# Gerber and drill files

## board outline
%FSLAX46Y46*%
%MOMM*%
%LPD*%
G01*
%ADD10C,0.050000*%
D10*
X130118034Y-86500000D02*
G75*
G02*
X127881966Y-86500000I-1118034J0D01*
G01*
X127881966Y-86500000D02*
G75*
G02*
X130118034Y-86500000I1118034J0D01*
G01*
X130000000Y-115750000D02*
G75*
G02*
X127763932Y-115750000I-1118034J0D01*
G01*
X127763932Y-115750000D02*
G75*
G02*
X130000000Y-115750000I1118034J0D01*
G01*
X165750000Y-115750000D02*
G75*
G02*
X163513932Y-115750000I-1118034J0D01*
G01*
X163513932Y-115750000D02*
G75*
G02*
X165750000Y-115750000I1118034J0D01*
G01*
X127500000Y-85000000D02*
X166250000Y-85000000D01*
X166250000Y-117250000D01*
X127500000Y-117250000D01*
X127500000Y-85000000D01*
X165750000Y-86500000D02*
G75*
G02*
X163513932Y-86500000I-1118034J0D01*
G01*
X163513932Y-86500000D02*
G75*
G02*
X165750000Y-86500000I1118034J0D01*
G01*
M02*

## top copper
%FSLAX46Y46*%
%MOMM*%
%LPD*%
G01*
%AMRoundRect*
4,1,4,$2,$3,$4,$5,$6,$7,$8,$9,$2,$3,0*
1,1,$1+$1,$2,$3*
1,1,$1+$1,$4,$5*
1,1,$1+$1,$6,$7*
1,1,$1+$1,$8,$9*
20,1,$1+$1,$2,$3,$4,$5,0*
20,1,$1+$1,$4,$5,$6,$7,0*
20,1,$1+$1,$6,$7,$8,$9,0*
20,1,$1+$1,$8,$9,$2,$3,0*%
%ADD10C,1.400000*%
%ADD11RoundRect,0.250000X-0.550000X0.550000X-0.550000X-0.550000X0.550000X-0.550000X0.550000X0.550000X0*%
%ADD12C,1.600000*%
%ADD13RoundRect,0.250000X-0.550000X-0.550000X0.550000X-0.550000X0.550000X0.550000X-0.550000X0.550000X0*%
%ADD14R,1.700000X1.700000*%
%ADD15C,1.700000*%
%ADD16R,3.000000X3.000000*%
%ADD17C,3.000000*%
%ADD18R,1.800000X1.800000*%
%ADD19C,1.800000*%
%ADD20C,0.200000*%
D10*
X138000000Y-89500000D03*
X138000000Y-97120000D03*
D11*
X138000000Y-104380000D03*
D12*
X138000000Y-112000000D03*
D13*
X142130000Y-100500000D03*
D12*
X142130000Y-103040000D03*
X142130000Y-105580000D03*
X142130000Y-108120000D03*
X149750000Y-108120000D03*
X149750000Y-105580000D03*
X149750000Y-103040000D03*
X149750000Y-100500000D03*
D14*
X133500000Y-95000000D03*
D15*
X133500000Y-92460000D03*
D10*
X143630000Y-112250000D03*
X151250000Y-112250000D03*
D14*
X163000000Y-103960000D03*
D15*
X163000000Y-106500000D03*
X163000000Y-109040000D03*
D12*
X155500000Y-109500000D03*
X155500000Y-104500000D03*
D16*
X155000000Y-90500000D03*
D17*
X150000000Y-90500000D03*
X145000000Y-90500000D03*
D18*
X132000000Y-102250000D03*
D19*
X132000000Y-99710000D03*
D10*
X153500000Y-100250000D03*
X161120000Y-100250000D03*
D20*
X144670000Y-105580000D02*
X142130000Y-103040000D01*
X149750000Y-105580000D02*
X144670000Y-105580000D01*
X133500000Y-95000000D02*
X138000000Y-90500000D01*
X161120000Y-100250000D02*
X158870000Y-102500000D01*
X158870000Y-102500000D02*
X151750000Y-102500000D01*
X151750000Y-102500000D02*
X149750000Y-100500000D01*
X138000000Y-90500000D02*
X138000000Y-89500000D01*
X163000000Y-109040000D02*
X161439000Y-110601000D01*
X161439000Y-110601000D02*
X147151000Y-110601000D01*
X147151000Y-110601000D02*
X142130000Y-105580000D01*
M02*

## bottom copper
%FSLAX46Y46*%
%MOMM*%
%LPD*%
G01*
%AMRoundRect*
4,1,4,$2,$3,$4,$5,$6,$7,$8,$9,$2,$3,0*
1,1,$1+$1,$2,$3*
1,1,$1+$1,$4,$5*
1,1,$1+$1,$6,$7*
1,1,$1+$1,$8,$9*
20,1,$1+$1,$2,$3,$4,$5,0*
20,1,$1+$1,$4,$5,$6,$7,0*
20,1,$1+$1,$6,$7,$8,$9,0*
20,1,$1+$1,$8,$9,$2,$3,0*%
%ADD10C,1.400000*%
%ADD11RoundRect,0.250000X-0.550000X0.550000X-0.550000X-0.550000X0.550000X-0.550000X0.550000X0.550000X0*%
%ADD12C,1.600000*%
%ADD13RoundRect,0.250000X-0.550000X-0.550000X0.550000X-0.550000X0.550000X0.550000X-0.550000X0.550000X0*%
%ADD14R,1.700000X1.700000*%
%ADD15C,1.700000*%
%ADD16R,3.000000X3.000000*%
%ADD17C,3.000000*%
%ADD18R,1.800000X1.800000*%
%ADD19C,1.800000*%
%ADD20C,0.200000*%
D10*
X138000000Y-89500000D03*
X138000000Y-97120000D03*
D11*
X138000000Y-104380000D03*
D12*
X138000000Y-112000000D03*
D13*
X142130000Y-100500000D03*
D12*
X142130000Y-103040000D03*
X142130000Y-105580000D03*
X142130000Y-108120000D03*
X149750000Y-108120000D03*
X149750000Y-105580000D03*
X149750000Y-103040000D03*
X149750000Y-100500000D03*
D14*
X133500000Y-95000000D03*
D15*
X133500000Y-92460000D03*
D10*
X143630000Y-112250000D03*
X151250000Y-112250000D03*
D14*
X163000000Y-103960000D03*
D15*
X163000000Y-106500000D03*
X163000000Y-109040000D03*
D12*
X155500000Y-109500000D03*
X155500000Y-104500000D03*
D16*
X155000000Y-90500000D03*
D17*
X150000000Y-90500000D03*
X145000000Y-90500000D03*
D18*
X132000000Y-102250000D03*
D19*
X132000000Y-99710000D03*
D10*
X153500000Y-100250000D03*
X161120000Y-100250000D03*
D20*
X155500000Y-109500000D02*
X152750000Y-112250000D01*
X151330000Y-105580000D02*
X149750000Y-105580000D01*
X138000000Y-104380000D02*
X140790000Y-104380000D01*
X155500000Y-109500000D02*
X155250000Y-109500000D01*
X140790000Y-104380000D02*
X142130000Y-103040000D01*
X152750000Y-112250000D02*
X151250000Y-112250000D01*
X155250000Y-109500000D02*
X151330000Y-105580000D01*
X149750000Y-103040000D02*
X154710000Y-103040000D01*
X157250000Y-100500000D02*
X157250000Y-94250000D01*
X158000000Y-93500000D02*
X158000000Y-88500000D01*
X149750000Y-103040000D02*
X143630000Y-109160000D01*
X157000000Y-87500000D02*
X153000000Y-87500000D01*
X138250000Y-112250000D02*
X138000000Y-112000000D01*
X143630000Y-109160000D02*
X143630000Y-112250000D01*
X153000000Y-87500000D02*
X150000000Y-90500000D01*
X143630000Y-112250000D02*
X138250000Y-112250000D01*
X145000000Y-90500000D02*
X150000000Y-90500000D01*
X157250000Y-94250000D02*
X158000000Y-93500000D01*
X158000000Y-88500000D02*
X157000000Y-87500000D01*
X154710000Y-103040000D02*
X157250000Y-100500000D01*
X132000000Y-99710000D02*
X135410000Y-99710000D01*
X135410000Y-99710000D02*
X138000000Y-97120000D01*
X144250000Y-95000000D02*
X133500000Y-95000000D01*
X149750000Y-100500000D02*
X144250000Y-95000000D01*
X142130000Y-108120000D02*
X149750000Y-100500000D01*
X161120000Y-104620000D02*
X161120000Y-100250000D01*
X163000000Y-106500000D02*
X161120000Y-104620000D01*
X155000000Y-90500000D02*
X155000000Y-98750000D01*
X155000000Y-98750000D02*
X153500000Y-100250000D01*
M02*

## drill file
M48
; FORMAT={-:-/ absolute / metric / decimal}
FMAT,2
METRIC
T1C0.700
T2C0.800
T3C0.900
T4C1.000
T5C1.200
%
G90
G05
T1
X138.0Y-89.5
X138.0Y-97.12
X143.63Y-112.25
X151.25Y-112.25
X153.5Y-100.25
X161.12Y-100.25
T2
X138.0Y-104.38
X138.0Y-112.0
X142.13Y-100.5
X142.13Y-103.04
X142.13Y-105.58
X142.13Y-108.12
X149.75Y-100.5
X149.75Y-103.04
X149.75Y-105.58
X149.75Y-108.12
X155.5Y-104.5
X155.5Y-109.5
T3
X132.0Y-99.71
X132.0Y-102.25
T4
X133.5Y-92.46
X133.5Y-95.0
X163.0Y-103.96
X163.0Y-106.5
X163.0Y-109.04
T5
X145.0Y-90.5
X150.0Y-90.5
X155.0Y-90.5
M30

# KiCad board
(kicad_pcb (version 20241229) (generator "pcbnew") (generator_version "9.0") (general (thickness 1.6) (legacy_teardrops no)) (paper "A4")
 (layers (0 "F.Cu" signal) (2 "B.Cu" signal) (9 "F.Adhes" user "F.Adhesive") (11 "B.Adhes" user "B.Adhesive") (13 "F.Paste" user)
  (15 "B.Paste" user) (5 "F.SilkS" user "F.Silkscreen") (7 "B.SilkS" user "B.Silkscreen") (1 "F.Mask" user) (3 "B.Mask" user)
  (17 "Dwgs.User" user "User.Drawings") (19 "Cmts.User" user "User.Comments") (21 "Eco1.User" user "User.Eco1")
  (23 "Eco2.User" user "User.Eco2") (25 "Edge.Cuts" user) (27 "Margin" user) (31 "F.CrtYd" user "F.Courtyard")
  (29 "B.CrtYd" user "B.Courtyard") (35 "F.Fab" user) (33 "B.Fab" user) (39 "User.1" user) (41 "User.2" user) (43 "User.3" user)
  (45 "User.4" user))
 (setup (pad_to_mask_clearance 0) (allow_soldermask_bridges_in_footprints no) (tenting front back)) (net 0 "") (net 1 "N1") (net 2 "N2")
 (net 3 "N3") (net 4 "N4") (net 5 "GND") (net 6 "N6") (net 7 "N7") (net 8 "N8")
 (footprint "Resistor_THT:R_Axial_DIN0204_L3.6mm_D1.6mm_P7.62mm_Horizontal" (layer "F.Cu") (at 138 89.5 -90)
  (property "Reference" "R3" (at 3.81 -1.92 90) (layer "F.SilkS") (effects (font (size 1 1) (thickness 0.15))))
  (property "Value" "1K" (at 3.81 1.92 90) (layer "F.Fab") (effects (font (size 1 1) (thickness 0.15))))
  (pad "1" thru_hole circle (at 0 0 270) (size 1.4 1.4) (drill 0.7) (layers "*.Cu" "*.Mask") (remove_unused_layers no) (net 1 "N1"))
  (pad "2" thru_hole circle (at 7.62 0 270) (size 1.4 1.4) (drill 0.7) (layers "*.Cu" "*.Mask") (remove_unused_layers no) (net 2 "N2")))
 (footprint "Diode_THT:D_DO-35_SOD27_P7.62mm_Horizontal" (layer "F.Cu") (at 138 104.38 -90)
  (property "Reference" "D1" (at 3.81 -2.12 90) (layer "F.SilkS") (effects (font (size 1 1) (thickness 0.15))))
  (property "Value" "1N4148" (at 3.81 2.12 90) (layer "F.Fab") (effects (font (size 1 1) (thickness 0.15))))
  (pad "1" thru_hole roundrect (at 0 0 270) (size 1.6 1.6) (drill 0.8) (layers "*.Cu" "*.Mask") (remove_unused_layers no)
   (roundrect_rratio 0.15625) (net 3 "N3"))
  (pad "2" thru_hole circle (at 7.62 0 270) (size 1.6 1.6) (drill 0.8) (layers "*.Cu" "*.Mask") (remove_unused_layers no) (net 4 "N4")))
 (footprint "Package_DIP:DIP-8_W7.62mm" (layer "F.Cu") (at 142.13 100.5)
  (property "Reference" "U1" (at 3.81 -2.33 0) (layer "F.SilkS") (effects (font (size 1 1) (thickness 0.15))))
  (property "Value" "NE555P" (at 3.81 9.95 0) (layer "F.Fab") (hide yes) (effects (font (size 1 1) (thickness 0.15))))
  (pad "1" thru_hole roundrect (at 0 0) (size 1.6 1.6) (drill 0.8) (layers "*.Cu" "*.Mask") (remove_unused_layers no)
   (roundrect_rratio 0.15625) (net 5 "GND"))
  (pad "2" thru_hole circle (at 0 2.54) (size 1.6 1.6) (drill 0.8) (layers "*.Cu" "*.Mask") (remove_unused_layers no) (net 3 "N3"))
  (pad "3" thru_hole circle (at 0 5.08) (size 1.6 1.6) (drill 0.8) (layers "*.Cu" "*.Mask") (remove_unused_layers no) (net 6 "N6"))
  (pad "4" thru_hole circle (at 0 7.62) (size 1.6 1.6) (drill 0.8) (layers "*.Cu" "*.Mask") (remove_unused_layers no) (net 1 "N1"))
  (pad "5" thru_hole circle (at 7.62 7.62) (size 1.6 1.6) (drill 0.8) (layers "*.Cu" "*.Mask") (remove_unused_layers no) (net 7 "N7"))
  (pad "6" thru_hole circle (at 7.62 5.08) (size 1.6 1.6) (drill 0.8) (layers "*.Cu" "*.Mask") (remove_unused_layers no) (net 3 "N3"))
  (pad "7" thru_hole circle (at 7.62 2.54) (size 1.6 1.6) (drill 0.8) (layers "*.Cu" "*.Mask") (remove_unused_layers no) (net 4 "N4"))
  (pad "8" thru_hole circle (at 7.62 0) (size 1.6 1.6) (drill 0.8) (layers "*.Cu" "*.Mask") (remove_unused_layers no) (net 1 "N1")))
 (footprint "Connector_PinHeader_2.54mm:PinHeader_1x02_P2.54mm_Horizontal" (layer "F.Cu") (at 133.5 95 180)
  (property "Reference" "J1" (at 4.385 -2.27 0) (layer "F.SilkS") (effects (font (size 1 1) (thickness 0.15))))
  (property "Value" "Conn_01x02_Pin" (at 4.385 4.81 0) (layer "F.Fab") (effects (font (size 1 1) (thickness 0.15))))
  (pad "1" thru_hole rect (at 0 0 180) (size 1.7 1.7) (drill 1) (layers "*.Cu" "*.Mask") (remove_unused_layers no) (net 1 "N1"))
  (pad "2" thru_hole circle (at 0 2.54 180) (size 1.7 1.7) (drill 1) (layers "*.Cu" "*.Mask") (remove_unused_layers no) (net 5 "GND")))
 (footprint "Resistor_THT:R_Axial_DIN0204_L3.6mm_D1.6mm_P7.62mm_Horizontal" (layer "F.Cu") (at 143.63 112.25)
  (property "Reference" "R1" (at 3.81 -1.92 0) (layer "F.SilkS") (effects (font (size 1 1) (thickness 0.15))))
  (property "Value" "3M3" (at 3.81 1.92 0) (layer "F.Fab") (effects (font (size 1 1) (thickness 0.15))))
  (pad "1" thru_hole circle (at 0 0) (size 1.4 1.4) (drill 0.7) (layers "*.Cu" "*.Mask") (remove_unused_layers no) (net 4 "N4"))
  (pad "2" thru_hole circle (at 7.62 0) (size 1.4 1.4) (drill 0.7) (layers "*.Cu" "*.Mask") (remove_unused_layers no) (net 3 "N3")))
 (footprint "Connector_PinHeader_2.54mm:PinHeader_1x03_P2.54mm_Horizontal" (layer "F.Cu") (at 163 103.96)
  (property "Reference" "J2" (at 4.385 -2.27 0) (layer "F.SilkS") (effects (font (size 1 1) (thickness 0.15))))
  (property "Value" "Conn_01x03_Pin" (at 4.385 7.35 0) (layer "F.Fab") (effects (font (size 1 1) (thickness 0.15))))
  (pad "1" thru_hole rect (at 0 0) (size 1.7 1.7) (drill 1) (layers "*.Cu" "*.Mask") (remove_unused_layers no) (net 5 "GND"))
  (pad "2" thru_hole circle (at 0 2.54) (size 1.7 1.7) (drill 1) (layers "*.Cu" "*.Mask") (remove_unused_layers no) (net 1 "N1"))
  (pad "3" thru_hole circle (at 0 5.08) (size 1.7 1.7) (drill 1) (layers "*.Cu" "*.Mask") (remove_unused_layers no) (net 6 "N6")))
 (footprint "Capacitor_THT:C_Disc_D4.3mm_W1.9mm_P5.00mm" (layer "F.Cu") (at 155.5 109.5 90)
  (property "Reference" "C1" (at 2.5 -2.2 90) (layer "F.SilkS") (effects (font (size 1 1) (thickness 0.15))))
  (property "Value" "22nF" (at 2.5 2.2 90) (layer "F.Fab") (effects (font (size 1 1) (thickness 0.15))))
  (pad "1" thru_hole circle (at 0 0 90) (size 1.6 1.6) (drill 0.8) (layers "*.Cu" "*.Mask") (remove_unused_layers no) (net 3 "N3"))
  (pad "2" thru_hole circle (at 5 0 90) (size 1.6 1.6) (drill 0.8) (layers "*.Cu" "*.Mask") (remove_unused_layers no) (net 5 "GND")))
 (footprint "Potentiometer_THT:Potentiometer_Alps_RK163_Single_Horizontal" (layer "F.Cu") (at 155 90.5 -90)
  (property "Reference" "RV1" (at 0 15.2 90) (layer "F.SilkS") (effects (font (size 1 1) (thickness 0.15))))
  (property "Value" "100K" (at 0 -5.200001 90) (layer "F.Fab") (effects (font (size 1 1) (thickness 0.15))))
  (pad "1" thru_hole rect (at 0 0 90) (size 3 3) (drill 1.2) (layers "*.Cu" "*.Mask") (remove_unused_layers no) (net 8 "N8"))
  (pad "2" thru_hole circle (at 0 5 90) (size 3 3) (drill 1.2) (layers "*.Cu" "*.Mask") (remove_unused_layers no) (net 4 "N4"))
  (pad "3" thru_hole circle (at 0 10 90) (size 3 3) (drill 1.2) (layers "*.Cu" "*.Mask") (remove_unused_layers no) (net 4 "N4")))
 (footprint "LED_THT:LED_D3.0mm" (layer "F.Cu") (at 132 102.25 90)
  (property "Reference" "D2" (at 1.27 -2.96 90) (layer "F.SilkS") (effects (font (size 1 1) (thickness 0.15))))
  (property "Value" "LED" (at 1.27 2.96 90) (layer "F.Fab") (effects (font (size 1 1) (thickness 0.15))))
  (pad "1" thru_hole rect (at 0 0 90) (size 1.8 1.8) (drill 0.9) (layers "*.Cu" "*.Mask") (remove_unused_layers no) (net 5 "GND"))
  (pad "2" thru_hole circle (at 2.54 0 90) (size 1.8 1.8) (drill 0.9) (layers "*.Cu" "*.Mask") (remove_unused_layers no) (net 2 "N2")))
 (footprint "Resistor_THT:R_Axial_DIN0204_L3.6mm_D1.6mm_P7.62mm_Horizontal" (layer "F.Cu") (at 153.5 100.25)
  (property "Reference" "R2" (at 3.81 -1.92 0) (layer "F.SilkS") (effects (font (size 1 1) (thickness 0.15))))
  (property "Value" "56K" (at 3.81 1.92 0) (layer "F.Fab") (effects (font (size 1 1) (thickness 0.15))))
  (pad "1" thru_hole circle (at 0 0) (size 1.4 1.4) (drill 0.7) (layers "*.Cu" "*.Mask") (remove_unused_layers no) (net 8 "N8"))
  (pad "2" thru_hole circle (at 7.62 0) (size 1.4 1.4) (drill 0.7) (layers "*.Cu" "*.Mask") (remove_unused_layers no) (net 1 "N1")))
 (gr_circle (center 129 86.5) (end 128 86) (stroke (width 0.05) (type default)) (fill no) (layer "Edge.Cuts"))
 (gr_circle (center 128.881966 115.75) (end 127.881966 115.25) (stroke (width 0.05) (type default)) (fill no) (layer "Edge.Cuts"))
 (gr_circle (center 164.631966 115.75) (end 163.631966 115.25) (stroke (width 0.05) (type default)) (fill no) (layer "Edge.Cuts"))
 (gr_rect (start 127.5 85) (end 166.25 117.25) (stroke (width 0.05) (type default)) (fill no) (layer "Edge.Cuts"))
 (gr_circle (center 164.631966 86.5) (end 163.631966 86) (stroke (width 0.05) (type default)) (fill no) (layer "Edge.Cuts"))
 (segment (start 144.67 105.58) (end 142.13 103.04) (width 0.2) (layer "F.Cu") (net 3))
 (segment (start 149.75 105.58) (end 144.67 105.58) (width 0.2) (layer "F.Cu") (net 3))
 (segment (start 155.5 109.5) (end 152.75 112.25) (width 0.2) (layer "B.Cu") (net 3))
 (segment (start 151.33 105.58) (end 149.75 105.58) (width 0.2) (layer "B.Cu") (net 3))
 (segment (start 138 104.38) (end 140.79 104.38) (width 0.2) (layer "B.Cu") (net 3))
 (segment (start 155.5 109.5) (end 155.25 109.5) (width 0.2) (layer "B.Cu") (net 3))
 (segment (start 140.79 104.38) (end 142.13 103.04) (width 0.2) (layer "B.Cu") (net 3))
 (segment (start 152.75 112.25) (end 151.25 112.25) (width 0.2) (layer "B.Cu") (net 3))
 (segment (start 155.25 109.5) (end 151.33 105.58) (width 0.2) (layer "B.Cu") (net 3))
 (segment (start 149.75 103.04) (end 154.71 103.04) (width 0.2) (layer "B.Cu") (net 4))
 (segment (start 157.25 100.5) (end 157.25 94.25) (width 0.2) (layer "B.Cu") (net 4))
 (segment (start 158 93.5) (end 158 88.5) (width 0.2) (layer "B.Cu") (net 4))
 (segment (start 149.75 103.04) (end 143.63 109.16) (width 0.2) (layer "B.Cu") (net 4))
 (segment (start 157 87.5) (end 153 87.5) (width 0.2) (layer "B.Cu") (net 4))
 (segment (start 138.25 112.25) (end 138 112) (width 0.2) (layer "B.Cu") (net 4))
 (segment (start 143.63 109.16) (end 143.63 112.25) (width 0.2) (layer "B.Cu") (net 4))
 (segment (start 153 87.5) (end 150 90.5) (width 0.2) (layer "B.Cu") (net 4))
 (segment (start 143.63 112.25) (end 138.25 112.25) (width 0.2) (layer "B.Cu") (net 4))
 (segment (start 145 90.5) (end 150 90.5) (width 0.2) (layer "B.Cu") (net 4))
 (segment (start 157.25 94.25) (end 158 93.5) (width 0.2) (layer "B.Cu") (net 4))
 (segment (start 158 88.5) (end 157 87.5) (width 0.2) (layer "B.Cu") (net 4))
 (segment (start 154.71 103.04) (end 157.25 100.5) (width 0.2) (layer "B.Cu") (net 4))
 (segment (start 132 99.71) (end 135.41 99.71) (width 0.2) (layer "B.Cu") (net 2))
 (segment (start 135.41 99.71) (end 138 97.12) (width 0.2) (layer "B.Cu") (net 2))
 (segment (start 133.5 95) (end 138 90.5) (width 0.2) (layer "F.Cu") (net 1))
 (segment (start 161.12 100.25) (end 158.87 102.5) (width 0.2) (layer "F.Cu") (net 1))
 (segment (start 158.87 102.5) (end 151.75 102.5) (width 0.2) (layer "F.Cu") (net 1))
 (segment (start 151.75 102.5) (end 149.75 100.5) (width 0.2) (layer "F.Cu") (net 1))
 (segment (start 138 90.5) (end 138 89.5) (width 0.2) (layer "F.Cu") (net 1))
 (segment (start 144.25 95) (end 133.5 95) (width 0.2) (layer "B.Cu") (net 1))
 (segment (start 149.75 100.5) (end 144.25 95) (width 0.2) (layer "B.Cu") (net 1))
 (segment (start 142.13 108.12) (end 149.75 100.5) (width 0.2) (layer "B.Cu") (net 1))
 (segment (start 161.12 104.62) (end 161.12 100.25) (width 0.2) (layer "B.Cu") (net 1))
 (segment (start 163 106.5) (end 161.12 104.62) (width 0.2) (layer "B.Cu") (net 1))
 (segment (start 163 109.04) (end 161.439 110.601) (width 0.2) (layer "F.Cu") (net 6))
 (segment (start 161.439 110.601) (end 147.151 110.601) (width 0.2) (layer "F.Cu") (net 6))
 (segment (start 147.151 110.601) (end 142.13 105.58) (width 0.2) (layer "F.Cu") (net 6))
 (segment (start 155 90.5) (end 155 98.75) (width 0.2) (layer "B.Cu") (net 8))
 (segment (start 155 98.75) (end 153.5 100.25) (width 0.2) (layer "B.Cu") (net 8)))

